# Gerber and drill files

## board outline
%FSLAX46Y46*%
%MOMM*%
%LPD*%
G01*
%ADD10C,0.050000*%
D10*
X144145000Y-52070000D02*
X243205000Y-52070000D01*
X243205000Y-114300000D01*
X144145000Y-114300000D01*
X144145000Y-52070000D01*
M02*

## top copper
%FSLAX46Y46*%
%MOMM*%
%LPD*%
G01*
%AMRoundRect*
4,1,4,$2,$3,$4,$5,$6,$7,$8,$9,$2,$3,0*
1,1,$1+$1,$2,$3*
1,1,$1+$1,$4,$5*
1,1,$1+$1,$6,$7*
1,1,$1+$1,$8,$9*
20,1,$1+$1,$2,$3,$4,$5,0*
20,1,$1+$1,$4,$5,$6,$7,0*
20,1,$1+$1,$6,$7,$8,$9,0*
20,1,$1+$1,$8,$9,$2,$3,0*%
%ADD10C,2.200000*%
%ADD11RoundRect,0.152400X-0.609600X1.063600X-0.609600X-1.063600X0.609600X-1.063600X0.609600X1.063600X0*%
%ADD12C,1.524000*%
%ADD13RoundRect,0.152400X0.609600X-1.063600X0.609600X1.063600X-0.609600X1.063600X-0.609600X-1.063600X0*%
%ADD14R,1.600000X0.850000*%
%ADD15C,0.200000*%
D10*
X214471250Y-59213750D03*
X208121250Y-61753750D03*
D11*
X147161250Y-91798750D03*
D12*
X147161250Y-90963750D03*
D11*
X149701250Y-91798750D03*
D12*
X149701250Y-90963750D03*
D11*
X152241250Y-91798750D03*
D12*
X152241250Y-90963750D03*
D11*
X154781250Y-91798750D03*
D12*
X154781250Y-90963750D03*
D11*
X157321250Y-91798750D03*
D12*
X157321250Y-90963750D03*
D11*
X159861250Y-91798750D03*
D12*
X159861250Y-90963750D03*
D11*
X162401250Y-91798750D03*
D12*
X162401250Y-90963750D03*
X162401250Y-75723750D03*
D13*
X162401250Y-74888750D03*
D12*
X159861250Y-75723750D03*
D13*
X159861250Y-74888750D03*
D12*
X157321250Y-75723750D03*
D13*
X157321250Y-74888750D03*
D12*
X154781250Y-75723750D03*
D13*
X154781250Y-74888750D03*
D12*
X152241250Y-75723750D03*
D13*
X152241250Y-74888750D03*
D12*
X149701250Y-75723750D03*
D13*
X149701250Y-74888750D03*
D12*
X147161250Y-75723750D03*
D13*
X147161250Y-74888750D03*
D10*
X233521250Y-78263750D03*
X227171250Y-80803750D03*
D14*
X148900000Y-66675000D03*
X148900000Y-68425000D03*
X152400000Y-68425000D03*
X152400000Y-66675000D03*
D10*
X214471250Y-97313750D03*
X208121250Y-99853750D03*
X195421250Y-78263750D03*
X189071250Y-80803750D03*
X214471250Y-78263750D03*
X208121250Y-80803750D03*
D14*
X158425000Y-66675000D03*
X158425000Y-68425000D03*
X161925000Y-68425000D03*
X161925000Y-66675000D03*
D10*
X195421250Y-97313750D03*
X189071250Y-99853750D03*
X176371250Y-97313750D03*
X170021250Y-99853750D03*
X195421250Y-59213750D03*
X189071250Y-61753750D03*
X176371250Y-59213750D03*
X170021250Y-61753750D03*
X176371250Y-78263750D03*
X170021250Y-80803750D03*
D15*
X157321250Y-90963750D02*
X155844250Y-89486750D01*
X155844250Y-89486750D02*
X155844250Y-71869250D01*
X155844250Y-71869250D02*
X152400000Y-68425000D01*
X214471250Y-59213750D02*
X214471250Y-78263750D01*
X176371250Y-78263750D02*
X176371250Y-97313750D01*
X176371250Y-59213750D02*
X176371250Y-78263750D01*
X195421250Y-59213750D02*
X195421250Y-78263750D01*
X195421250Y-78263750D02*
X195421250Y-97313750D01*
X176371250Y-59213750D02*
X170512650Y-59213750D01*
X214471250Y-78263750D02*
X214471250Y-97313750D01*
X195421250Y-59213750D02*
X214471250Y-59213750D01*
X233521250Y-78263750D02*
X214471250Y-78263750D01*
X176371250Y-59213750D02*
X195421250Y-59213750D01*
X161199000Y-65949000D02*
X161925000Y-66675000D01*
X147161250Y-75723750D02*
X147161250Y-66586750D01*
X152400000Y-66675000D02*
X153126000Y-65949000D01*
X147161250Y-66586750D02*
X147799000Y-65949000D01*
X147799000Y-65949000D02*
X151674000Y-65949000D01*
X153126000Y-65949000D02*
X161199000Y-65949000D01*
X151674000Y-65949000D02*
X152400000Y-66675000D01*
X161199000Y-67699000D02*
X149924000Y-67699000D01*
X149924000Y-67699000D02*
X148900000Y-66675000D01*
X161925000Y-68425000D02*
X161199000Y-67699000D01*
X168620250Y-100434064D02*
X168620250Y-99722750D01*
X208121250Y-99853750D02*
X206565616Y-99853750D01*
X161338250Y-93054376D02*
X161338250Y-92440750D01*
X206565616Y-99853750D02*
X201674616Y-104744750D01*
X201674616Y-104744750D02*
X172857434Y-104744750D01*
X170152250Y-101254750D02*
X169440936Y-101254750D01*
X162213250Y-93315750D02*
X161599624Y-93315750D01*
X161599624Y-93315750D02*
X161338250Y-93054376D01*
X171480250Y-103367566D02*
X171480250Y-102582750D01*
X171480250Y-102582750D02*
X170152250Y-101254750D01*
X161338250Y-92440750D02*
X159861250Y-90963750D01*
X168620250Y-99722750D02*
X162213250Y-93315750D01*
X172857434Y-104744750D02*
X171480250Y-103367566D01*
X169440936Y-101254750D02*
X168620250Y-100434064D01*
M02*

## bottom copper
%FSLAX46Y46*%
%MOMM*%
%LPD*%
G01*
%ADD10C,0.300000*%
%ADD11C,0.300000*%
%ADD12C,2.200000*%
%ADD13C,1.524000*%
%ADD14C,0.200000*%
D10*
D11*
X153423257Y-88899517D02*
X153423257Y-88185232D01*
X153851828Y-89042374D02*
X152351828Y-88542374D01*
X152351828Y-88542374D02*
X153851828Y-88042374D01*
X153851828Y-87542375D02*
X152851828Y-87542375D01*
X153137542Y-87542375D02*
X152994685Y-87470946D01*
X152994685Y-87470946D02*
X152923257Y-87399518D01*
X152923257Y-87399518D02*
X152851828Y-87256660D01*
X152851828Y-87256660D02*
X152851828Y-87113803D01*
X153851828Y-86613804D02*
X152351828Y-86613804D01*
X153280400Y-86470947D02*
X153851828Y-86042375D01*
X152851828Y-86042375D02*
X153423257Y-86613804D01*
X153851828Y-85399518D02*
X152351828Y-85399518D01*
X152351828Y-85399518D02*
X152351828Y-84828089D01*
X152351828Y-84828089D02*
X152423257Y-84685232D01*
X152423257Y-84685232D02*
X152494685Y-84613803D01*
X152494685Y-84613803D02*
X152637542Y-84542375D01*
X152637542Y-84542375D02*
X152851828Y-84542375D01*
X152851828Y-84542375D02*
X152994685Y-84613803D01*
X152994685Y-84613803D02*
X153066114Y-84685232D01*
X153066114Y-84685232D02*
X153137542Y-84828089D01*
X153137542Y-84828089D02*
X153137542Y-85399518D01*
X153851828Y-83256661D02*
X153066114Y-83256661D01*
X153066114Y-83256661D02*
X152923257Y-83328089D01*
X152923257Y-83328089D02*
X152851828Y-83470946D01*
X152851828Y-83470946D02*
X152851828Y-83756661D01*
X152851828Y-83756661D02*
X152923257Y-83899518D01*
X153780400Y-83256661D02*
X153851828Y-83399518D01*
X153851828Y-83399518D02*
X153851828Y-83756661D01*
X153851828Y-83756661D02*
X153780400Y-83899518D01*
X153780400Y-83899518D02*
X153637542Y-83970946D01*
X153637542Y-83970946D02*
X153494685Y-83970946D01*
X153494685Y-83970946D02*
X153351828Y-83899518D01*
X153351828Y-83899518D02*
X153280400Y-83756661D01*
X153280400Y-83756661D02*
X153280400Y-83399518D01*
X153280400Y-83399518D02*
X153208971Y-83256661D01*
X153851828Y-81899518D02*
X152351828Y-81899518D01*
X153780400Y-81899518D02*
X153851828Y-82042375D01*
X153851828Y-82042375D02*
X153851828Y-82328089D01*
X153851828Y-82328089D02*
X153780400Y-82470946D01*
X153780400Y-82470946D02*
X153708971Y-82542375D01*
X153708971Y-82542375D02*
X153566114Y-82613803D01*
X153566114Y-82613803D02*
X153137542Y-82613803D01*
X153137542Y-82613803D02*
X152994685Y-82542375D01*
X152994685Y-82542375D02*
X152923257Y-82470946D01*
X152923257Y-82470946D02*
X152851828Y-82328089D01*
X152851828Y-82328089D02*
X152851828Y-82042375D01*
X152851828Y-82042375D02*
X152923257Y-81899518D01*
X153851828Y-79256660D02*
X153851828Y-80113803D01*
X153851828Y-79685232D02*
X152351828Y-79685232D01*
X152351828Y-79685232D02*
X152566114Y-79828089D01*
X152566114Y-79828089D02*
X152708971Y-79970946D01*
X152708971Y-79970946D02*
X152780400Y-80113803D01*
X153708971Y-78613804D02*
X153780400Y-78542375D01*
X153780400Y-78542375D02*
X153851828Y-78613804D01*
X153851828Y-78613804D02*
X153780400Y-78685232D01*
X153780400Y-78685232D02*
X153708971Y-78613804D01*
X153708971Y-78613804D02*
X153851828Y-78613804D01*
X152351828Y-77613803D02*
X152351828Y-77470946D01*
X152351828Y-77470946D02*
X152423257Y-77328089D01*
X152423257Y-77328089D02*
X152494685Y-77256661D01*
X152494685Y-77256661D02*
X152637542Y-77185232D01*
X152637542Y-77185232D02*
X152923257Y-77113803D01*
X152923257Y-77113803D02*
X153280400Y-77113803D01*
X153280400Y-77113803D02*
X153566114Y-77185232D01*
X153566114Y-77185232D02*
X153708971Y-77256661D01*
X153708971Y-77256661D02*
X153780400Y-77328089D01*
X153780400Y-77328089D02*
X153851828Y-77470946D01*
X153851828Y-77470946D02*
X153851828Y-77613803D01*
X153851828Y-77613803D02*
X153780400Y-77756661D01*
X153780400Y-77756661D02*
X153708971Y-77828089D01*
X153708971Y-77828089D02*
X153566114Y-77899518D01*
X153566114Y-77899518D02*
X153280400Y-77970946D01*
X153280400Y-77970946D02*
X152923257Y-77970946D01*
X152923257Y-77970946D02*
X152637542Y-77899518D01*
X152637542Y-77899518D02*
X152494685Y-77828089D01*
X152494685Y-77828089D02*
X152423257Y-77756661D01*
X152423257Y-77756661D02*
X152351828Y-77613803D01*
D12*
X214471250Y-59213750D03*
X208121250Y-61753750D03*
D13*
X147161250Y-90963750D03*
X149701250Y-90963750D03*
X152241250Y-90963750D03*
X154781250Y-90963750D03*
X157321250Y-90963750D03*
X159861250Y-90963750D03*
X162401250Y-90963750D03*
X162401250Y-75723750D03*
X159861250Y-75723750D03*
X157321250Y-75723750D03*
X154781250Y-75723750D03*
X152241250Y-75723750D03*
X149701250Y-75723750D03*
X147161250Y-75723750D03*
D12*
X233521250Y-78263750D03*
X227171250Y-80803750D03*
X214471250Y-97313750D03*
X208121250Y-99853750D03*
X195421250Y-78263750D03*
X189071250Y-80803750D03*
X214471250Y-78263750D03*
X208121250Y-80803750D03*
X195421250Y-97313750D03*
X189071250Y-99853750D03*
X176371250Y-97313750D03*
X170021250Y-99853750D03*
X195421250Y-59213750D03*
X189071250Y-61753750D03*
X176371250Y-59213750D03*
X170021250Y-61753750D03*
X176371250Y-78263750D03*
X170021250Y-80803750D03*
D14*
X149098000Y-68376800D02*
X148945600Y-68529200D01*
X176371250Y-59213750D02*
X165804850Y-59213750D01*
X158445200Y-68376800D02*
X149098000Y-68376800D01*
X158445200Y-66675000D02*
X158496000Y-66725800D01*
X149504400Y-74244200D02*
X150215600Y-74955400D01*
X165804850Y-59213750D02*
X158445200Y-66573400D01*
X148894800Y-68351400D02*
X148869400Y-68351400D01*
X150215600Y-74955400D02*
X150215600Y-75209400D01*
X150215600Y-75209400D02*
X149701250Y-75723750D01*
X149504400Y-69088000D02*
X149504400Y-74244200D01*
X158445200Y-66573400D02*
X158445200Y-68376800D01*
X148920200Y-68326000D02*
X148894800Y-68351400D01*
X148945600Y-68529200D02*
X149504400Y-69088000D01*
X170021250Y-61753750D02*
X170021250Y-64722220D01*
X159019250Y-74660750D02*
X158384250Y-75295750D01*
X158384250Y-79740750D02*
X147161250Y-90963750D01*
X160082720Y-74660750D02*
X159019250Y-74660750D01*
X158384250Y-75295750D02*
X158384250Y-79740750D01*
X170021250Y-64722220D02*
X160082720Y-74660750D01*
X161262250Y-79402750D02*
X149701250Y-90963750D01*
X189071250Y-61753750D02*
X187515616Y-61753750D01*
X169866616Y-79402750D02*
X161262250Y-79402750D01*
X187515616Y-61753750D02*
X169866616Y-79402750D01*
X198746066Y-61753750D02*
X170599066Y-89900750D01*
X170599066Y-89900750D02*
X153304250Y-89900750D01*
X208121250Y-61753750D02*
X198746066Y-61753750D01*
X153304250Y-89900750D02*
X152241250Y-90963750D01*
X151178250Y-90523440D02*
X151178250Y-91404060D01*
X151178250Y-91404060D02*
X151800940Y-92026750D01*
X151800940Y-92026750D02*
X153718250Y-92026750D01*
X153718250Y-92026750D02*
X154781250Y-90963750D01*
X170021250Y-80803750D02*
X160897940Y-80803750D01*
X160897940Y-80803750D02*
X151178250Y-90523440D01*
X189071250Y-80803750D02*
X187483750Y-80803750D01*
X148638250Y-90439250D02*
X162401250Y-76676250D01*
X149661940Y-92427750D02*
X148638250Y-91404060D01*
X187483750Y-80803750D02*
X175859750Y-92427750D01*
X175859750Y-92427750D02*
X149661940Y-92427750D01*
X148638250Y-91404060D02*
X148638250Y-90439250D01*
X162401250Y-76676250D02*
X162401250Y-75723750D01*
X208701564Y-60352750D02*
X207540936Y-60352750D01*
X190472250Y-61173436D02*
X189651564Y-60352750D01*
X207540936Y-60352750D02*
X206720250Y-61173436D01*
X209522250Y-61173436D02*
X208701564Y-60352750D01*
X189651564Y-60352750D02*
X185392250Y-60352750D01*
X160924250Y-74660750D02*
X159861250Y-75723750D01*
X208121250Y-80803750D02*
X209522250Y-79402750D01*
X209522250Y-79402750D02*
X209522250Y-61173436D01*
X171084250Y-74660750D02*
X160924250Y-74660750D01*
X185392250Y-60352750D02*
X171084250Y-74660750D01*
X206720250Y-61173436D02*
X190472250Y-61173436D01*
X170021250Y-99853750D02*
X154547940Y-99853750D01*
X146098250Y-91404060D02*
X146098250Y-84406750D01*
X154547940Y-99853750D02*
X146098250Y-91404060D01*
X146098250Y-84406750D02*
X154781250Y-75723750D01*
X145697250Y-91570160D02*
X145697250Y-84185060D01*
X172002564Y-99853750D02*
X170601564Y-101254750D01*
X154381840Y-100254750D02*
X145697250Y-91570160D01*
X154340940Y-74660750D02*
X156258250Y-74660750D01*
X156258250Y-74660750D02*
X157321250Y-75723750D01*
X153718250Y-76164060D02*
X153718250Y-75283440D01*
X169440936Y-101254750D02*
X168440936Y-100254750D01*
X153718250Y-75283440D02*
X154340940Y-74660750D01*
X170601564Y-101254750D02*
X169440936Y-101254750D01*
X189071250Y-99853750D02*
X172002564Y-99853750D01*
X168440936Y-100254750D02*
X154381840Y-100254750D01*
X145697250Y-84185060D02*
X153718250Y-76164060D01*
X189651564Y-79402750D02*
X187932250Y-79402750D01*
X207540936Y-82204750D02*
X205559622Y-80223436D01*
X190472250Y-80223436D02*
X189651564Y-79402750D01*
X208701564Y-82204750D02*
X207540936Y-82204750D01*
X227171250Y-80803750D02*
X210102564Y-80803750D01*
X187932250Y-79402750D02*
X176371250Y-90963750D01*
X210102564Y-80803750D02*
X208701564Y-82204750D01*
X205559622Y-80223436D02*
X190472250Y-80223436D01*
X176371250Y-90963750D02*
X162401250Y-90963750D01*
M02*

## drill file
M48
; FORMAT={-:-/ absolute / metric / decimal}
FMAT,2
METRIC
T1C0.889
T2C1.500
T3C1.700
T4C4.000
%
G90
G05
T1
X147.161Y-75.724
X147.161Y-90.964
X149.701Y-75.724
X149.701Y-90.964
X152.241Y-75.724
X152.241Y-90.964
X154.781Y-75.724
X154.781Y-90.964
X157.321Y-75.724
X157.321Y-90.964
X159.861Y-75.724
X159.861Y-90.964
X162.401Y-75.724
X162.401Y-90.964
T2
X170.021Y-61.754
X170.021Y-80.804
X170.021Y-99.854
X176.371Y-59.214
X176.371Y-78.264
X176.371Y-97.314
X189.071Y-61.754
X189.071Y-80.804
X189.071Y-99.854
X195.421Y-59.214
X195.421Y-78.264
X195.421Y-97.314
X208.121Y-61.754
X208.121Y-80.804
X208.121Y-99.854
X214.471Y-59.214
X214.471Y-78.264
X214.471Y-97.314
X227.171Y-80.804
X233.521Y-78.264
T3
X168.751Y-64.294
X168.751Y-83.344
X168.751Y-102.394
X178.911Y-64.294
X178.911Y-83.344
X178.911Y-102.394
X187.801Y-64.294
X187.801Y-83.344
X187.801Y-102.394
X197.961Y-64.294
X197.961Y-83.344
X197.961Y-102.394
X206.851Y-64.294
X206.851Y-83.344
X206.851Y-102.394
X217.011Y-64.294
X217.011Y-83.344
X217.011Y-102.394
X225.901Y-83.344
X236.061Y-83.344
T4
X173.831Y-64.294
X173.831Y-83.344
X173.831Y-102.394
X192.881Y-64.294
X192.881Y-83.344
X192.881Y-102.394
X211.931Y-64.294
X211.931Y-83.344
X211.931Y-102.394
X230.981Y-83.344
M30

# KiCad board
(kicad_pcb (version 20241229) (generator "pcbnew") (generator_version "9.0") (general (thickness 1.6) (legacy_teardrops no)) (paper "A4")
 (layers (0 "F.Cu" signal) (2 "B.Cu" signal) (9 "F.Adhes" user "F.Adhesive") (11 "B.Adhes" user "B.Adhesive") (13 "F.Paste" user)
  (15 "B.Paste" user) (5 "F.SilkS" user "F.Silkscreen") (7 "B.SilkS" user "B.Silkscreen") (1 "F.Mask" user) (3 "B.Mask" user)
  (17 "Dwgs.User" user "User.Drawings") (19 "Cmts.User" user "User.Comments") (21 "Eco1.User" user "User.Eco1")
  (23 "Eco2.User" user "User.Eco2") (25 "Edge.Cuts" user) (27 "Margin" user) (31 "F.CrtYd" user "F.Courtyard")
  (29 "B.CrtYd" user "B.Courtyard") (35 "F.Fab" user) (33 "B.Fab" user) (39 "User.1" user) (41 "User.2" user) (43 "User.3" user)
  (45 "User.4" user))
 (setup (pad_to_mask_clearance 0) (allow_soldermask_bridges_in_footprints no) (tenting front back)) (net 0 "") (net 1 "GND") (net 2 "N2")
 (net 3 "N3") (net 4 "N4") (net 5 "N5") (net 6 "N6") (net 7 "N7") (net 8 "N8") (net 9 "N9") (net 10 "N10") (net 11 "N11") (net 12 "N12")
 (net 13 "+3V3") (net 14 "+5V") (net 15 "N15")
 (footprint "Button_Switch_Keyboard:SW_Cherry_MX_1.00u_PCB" (layer "F.Cu") (at 214.47125 59.21375)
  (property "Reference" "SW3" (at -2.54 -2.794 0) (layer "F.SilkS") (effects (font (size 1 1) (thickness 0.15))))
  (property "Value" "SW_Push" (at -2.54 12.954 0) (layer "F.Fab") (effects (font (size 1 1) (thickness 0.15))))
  (pad "" np_thru_hole circle (at -7.62 5.08) (size 1.7 1.7) (drill 1.7) (layers "*.Cu" "*.Mask"))
  (pad "" np_thru_hole circle (at -2.54 5.08) (size 4 4) (drill 4) (layers "*.Cu" "*.Mask"))
  (pad "" np_thru_hole circle (at 2.54 5.08) (size 1.7 1.7) (drill 1.7) (layers "*.Cu" "*.Mask"))
  (pad "1" thru_hole circle (at 0 0) (size 2.2 2.2) (drill 1.5) (layers "*.Cu" "*.Mask") (remove_unused_layers no) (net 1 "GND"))
  (pad "2" thru_hole circle (at -6.35 2.54) (size 2.2 2.2) (drill 1.5) (layers "*.Cu" "*.Mask") (remove_unused_layers no) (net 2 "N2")))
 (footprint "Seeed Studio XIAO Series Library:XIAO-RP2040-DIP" (layer "F.Cu") (at 154.78125 83.34375 90)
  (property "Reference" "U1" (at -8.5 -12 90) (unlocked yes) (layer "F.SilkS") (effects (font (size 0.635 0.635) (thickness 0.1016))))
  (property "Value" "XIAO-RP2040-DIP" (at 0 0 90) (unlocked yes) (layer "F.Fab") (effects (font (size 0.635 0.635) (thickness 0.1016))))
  (pad "1" smd roundrect (at -8.455 -7.62 270) (size 2.432 1.524) (layers "F.Cu" "F.Mask") (roundrect_rratio 0.1) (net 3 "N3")
   (thermal_bridge_angle 45))
  (pad "1" thru_hole circle (at -7.62 -7.62 270) (size 1.524 1.524) (drill 0.889) (layers "*.Cu" "*.Mask") (remove_unused_layers no)
   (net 3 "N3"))
  (pad "2" smd roundrect (at -8.455 -5.08 270) (size 2.432 1.524) (layers "F.Cu" "F.Mask") (roundrect_rratio 0.1) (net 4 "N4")
   (thermal_bridge_angle 45))
  (pad "2" thru_hole circle (at -7.62 -5.08 270) (size 1.524 1.524) (drill 0.889) (layers "*.Cu" "*.Mask") (remove_unused_layers no)
   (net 4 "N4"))
  (pad "3" smd roundrect (at -8.455 -2.54 270) (size 2.432 1.524) (layers "F.Cu" "F.Mask") (roundrect_rratio 0.1) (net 2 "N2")
   (thermal_bridge_angle 45))
  (pad "3" thru_hole circle (at -7.62 -2.54 270) (size 1.524 1.524) (drill 0.889) (layers "*.Cu" "*.Mask") (remove_unused_layers no)
   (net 2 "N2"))
  (pad "4" smd roundrect (at -8.455 0 270) (size 2.432 1.524) (layers "F.Cu" "F.Mask") (roundrect_rratio 0.1) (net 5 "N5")
   (thermal_bridge_angle 45))
  (pad "4" thru_hole circle (at -7.62 0 270) (size 1.524 1.524) (drill 0.889) (layers "*.Cu" "*.Mask") (remove_unused_layers no)
   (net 5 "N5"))
  (pad "5" smd roundrect (at -8.455 2.54 270) (size 2.432 1.524) (layers "F.Cu" "F.Mask") (roundrect_rratio 0.1) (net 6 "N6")
   (thermal_bridge_angle 45))
  (pad "5" thru_hole circle (at -7.62 2.54 270) (size 1.524 1.524) (drill 0.889) (layers "*.Cu" "*.Mask") (remove_unused_layers no)
   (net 6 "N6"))
  (pad "6" smd roundrect (at -8.455 5.08 270) (size 2.432 1.524) (layers "F.Cu" "F.Mask") (roundrect_rratio 0.1) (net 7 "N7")
   (thermal_bridge_angle 45))
  (pad "6" thru_hole circle (at -7.62 5.08 270) (size 1.524 1.524) (drill 0.889) (layers "*.Cu" "*.Mask") (remove_unused_layers no)
   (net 7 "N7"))
  (pad "7" smd roundrect (at -8.455 7.62 270) (size 2.432 1.524) (layers "F.Cu" "F.Mask") (roundrect_rratio 0.1) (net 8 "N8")
   (thermal_bridge_angle 45))
  (pad "7" thru_hole circle (at -7.62 7.62 270) (size 1.524 1.524) (drill 0.889) (layers "*.Cu" "*.Mask") (remove_unused_layers no)
   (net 8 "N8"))
  (pad "8" thru_hole circle (at 7.62 7.62 90) (size 1.524 1.524) (drill 0.889) (layers "*.Cu" "*.Mask") (remove_unused_layers no)
   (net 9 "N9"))
  (pad "8" smd roundrect (at 8.455 7.62 90) (size 2.432 1.524) (layers "F.Cu" "F.Mask") (roundrect_rratio 0.1) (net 9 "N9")
   (thermal_bridge_angle 45))
  (pad "9" thru_hole circle (at 7.62 5.08 90) (size 1.524 1.524) (drill 0.889) (layers "*.Cu" "*.Mask") (remove_unused_layers no)
   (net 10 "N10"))
  (pad "9" smd roundrect (at 8.455 5.08 90) (size 2.432 1.524) (layers "F.Cu" "F.Mask") (roundrect_rratio 0.1) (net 10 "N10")
   (thermal_bridge_angle 45))
  (pad "10" thru_hole circle (at 7.62 2.54 90) (size 1.524 1.524) (drill 0.889) (layers "*.Cu" "*.Mask") (remove_unused_layers no)
   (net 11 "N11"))
  (pad "10" smd roundrect (at 8.455 2.54 90) (size 2.432 1.524) (layers "F.Cu" "F.Mask") (roundrect_rratio 0.1) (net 11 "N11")
   (thermal_bridge_angle 45))
  (pad "11" thru_hole circle (at 7.62 0 90) (size 1.524 1.524) (drill 0.889) (layers "*.Cu" "*.Mask") (remove_unused_layers no)
   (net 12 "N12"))
  (pad "11" smd roundrect (at 8.455 0 90) (size 2.432 1.524) (layers "F.Cu" "F.Mask") (roundrect_rratio 0.1) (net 12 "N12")
   (thermal_bridge_angle 45))
  (pad "12" thru_hole circle (at 7.62 -2.54 90) (size 1.524 1.524) (drill 0.889) (layers "*.Cu" "*.Mask") (remove_unused_layers no)
   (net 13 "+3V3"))
  (pad "12" smd roundrect (at 8.455 -2.54 90) (size 2.432 1.524) (layers "F.Cu" "F.Mask") (roundrect_rratio 0.1) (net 13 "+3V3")
   (thermal_bridge_angle 45))
  (pad "13" thru_hole circle (at 7.62 -5.08 90) (size 1.524 1.524) (drill 0.889) (layers "*.Cu" "*.Mask") (remove_unused_layers no)
   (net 1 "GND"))
  (pad "13" smd roundrect (at 8.455 -5.08 90) (size 2.432 1.524) (layers "F.Cu" "F.Mask") (roundrect_rratio 0.1) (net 1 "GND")
   (thermal_bridge_angle 45))
  (pad "14" thru_hole circle (at 7.62 -7.62 90) (size 1.524 1.524) (drill 0.889) (layers "*.Cu" "*.Mask") (remove_unused_layers no)
   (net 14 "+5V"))
  (pad "14" smd roundrect (at 8.455 -7.62 90) (size 2.432 1.524) (layers "F.Cu" "F.Mask") (roundrect_rratio 0.1) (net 14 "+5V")
   (thermal_bridge_angle 45)))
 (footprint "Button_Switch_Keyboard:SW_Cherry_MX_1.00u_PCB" (layer "F.Cu") (at 233.52125 78.26375)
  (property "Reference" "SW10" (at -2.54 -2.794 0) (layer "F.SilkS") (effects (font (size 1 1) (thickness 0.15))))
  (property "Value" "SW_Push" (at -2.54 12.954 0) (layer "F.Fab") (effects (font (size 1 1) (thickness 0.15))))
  (pad "" np_thru_hole circle (at -7.62 5.08) (size 1.7 1.7) (drill 1.7) (layers "*.Cu" "*.Mask"))
  (pad "" np_thru_hole circle (at -2.54 5.08) (size 4 4) (drill 4) (layers "*.Cu" "*.Mask"))
  (pad "" np_thru_hole circle (at 2.54 5.08) (size 1.7 1.7) (drill 1.7) (layers "*.Cu" "*.Mask"))
  (pad "1" thru_hole circle (at 0 0) (size 2.2 2.2) (drill 1.5) (layers "*.Cu" "*.Mask") (remove_unused_layers no) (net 1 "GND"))
  (pad "2" thru_hole circle (at -6.35 2.54) (size 2.2 2.2) (drill 1.5) (layers "*.Cu" "*.Mask") (remove_unused_layers no) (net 8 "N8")))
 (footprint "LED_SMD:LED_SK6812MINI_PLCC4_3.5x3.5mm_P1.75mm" (layer "F.Cu") (at 150.65 67.55)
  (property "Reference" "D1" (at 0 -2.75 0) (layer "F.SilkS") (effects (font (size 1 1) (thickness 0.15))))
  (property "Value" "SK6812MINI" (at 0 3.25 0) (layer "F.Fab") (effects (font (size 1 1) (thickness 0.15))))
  (pad "1" smd rect (at -1.75 -0.875) (size 1.6 0.85) (layers "F.Cu" "F.Mask" "F.Paste") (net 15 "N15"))
  (pad "2" smd rect (at -1.75 0.875) (size 1.6 0.85) (layers "F.Cu" "F.Mask" "F.Paste") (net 1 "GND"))
  (pad "3" smd rect (at 1.75 0.875) (size 1.6 0.85) (layers "F.Cu" "F.Mask" "F.Paste") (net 6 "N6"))
  (pad "4" smd rect (at 1.75 -0.875) (size 1.6 0.85) (layers "F.Cu" "F.Mask" "F.Paste") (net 14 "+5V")))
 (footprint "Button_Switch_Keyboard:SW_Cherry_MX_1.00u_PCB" (layer "F.Cu") (at 214.47125 97.31375)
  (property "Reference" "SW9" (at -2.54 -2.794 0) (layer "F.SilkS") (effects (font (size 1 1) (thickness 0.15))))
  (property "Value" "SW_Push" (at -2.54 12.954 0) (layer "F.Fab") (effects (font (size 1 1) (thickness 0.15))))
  (pad "" np_thru_hole circle (at -7.62 5.08) (size 1.7 1.7) (drill 1.7) (layers "*.Cu" "*.Mask"))
  (pad "" np_thru_hole circle (at -2.54 5.08) (size 4 4) (drill 4) (layers "*.Cu" "*.Mask"))
  (pad "" np_thru_hole circle (at 2.54 5.08) (size 1.7 1.7) (drill 1.7) (layers "*.Cu" "*.Mask"))
  (pad "1" thru_hole circle (at 0 0) (size 2.2 2.2) (drill 1.5) (layers "*.Cu" "*.Mask") (remove_unused_layers no) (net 1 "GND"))
  (pad "2" thru_hole circle (at -6.35 2.54) (size 2.2 2.2) (drill 1.5) (layers "*.Cu" "*.Mask") (remove_unused_layers no) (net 7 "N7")))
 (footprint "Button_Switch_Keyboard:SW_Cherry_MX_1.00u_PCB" (layer "F.Cu") (at 195.42125 78.26375)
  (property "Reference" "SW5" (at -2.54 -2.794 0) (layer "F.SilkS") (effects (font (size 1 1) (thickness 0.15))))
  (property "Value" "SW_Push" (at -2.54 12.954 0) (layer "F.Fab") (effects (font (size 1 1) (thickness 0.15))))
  (pad "" np_thru_hole circle (at -7.62 5.08) (size 1.7 1.7) (drill 1.7) (layers "*.Cu" "*.Mask"))
  (pad "" np_thru_hole circle (at -2.54 5.08) (size 4 4) (drill 4) (layers "*.Cu" "*.Mask"))
  (pad "" np_thru_hole circle (at 2.54 5.08) (size 1.7 1.7) (drill 1.7) (layers "*.Cu" "*.Mask"))
  (pad "1" thru_hole circle (at 0 0) (size 2.2 2.2) (drill 1.5) (layers "*.Cu" "*.Mask") (remove_unused_layers no) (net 1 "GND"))
  (pad "2" thru_hole circle (at -6.35 2.54) (size 2.2 2.2) (drill 1.5) (layers "*.Cu" "*.Mask") (remove_unused_layers no) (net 9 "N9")))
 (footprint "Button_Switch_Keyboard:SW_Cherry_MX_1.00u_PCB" (layer "F.Cu") (at 214.47125 78.26375)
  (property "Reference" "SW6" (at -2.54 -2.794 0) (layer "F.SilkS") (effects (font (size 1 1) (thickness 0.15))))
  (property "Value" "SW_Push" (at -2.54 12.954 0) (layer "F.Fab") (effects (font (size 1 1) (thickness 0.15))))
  (pad "" np_thru_hole circle (at -7.62 5.08) (size 1.7 1.7) (drill 1.7) (layers "*.Cu" "*.Mask"))
  (pad "" np_thru_hole circle (at -2.54 5.08) (size 4 4) (drill 4) (layers "*.Cu" "*.Mask"))
  (pad "" np_thru_hole circle (at 2.54 5.08) (size 1.7 1.7) (drill 1.7) (layers "*.Cu" "*.Mask"))
  (pad "1" thru_hole circle (at 0 0) (size 2.2 2.2) (drill 1.5) (layers "*.Cu" "*.Mask") (remove_unused_layers no) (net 1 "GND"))
  (pad "2" thru_hole circle (at -6.35 2.54) (size 2.2 2.2) (drill 1.5) (layers "*.Cu" "*.Mask") (remove_unused_layers no) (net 10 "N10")))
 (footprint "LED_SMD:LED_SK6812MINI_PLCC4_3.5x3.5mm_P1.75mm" (layer "F.Cu") (at 160.175 67.55)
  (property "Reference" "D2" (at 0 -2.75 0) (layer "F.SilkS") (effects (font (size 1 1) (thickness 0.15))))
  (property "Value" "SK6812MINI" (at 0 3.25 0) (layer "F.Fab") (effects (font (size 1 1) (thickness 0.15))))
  (pad "1" smd rect (at -1.75 -0.875) (size 1.6 0.85) (layers "F.Cu" "F.Mask" "F.Paste") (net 1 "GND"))
  (pad "2" smd rect (at -1.75 0.875) (size 1.6 0.85) (layers "F.Cu" "F.Mask" "F.Paste") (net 1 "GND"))
  (pad "3" smd rect (at 1.75 0.875) (size 1.6 0.85) (layers "F.Cu" "F.Mask" "F.Paste") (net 15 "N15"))
  (pad "4" smd rect (at 1.75 -0.875) (size 1.6 0.85) (layers "F.Cu" "F.Mask" "F.Paste") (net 14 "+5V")))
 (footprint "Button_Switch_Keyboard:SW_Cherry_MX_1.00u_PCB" (layer "F.Cu") (at 195.42125 97.31375)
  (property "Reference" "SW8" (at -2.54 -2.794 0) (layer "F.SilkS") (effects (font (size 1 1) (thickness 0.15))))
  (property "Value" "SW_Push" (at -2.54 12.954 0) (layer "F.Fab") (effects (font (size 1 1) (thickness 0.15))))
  (pad "" np_thru_hole circle (at -7.62 5.08) (size 1.7 1.7) (drill 1.7) (layers "*.Cu" "*.Mask"))
  (pad "" np_thru_hole circle (at -2.54 5.08) (size 4 4) (drill 4) (layers "*.Cu" "*.Mask"))
  (pad "" np_thru_hole circle (at 2.54 5.08) (size 1.7 1.7) (drill 1.7) (layers "*.Cu" "*.Mask"))
  (pad "1" thru_hole circle (at 0 0) (size 2.2 2.2) (drill 1.5) (layers "*.Cu" "*.Mask") (remove_unused_layers no) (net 1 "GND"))
  (pad "2" thru_hole circle (at -6.35 2.54) (size 2.2 2.2) (drill 1.5) (layers "*.Cu" "*.Mask") (remove_unused_layers no) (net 11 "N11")))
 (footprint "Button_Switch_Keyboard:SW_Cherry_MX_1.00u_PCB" (layer "F.Cu") (at 176.37125 97.31375)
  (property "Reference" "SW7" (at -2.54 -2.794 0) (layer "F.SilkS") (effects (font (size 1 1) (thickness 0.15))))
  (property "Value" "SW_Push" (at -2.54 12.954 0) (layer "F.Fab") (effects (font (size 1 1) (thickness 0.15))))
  (pad "" np_thru_hole circle (at -7.62 5.08) (size 1.7 1.7) (drill 1.7) (layers "*.Cu" "*.Mask"))
  (pad "" np_thru_hole circle (at -2.54 5.08) (size 4 4) (drill 4) (layers "*.Cu" "*.Mask"))
  (pad "" np_thru_hole circle (at 2.54 5.08) (size 1.7 1.7) (drill 1.7) (layers "*.Cu" "*.Mask"))
  (pad "1" thru_hole circle (at 0 0) (size 2.2 2.2) (drill 1.5) (layers "*.Cu" "*.Mask") (remove_unused_layers no) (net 1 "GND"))
  (pad "2" thru_hole circle (at -6.35 2.54) (size 2.2 2.2) (drill 1.5) (layers "*.Cu" "*.Mask") (remove_unused_layers no) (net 12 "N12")))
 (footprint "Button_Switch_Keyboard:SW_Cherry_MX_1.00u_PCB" (layer "F.Cu") (at 195.42125 59.21375)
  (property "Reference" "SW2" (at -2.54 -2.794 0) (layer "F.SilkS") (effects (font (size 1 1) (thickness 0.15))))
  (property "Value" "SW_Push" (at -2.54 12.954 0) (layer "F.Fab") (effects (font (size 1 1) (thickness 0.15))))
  (pad "" np_thru_hole circle (at -7.62 5.08) (size 1.7 1.7) (drill 1.7) (layers "*.Cu" "*.Mask"))
  (pad "" np_thru_hole circle (at -2.54 5.08) (size 4 4) (drill 4) (layers "*.Cu" "*.Mask"))
  (pad "" np_thru_hole circle (at 2.54 5.08) (size 1.7 1.7) (drill 1.7) (layers "*.Cu" "*.Mask"))
  (pad "1" thru_hole circle (at 0 0) (size 2.2 2.2) (drill 1.5) (layers "*.Cu" "*.Mask") (remove_unused_layers no) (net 1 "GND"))
  (pad "2" thru_hole circle (at -6.35 2.54) (size 2.2 2.2) (drill 1.5) (layers "*.Cu" "*.Mask") (remove_unused_layers no) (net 4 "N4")))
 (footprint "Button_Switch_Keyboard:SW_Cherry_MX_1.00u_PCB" (layer "F.Cu") (at 176.37125 59.21375)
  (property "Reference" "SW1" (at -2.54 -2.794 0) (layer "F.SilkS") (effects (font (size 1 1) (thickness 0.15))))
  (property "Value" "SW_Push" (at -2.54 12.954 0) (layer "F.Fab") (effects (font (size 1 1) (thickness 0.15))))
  (pad "" np_thru_hole circle (at -7.62 5.08) (size 1.7 1.7) (drill 1.7) (layers "*.Cu" "*.Mask"))
  (pad "" np_thru_hole circle (at -2.54 5.08) (size 4 4) (drill 4) (layers "*.Cu" "*.Mask"))
  (pad "" np_thru_hole circle (at 2.54 5.08) (size 1.7 1.7) (drill 1.7) (layers "*.Cu" "*.Mask"))
  (pad "1" thru_hole circle (at 0 0) (size 2.2 2.2) (drill 1.5) (layers "*.Cu" "*.Mask") (remove_unused_layers no) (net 1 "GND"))
  (pad "2" thru_hole circle (at -6.35 2.54) (size 2.2 2.2) (drill 1.5) (layers "*.Cu" "*.Mask") (remove_unused_layers no) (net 3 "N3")))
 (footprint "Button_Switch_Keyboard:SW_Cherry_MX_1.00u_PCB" (layer "F.Cu") (at 176.37125 78.26375)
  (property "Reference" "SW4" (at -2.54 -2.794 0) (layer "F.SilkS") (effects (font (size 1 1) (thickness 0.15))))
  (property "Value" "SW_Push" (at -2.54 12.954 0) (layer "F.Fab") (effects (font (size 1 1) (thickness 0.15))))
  (pad "" np_thru_hole circle (at -7.62 5.08) (size 1.7 1.7) (drill 1.7) (layers "*.Cu" "*.Mask"))
  (pad "" np_thru_hole circle (at -2.54 5.08) (size 4 4) (drill 4) (layers "*.Cu" "*.Mask"))
  (pad "" np_thru_hole circle (at 2.54 5.08) (size 1.7 1.7) (drill 1.7) (layers "*.Cu" "*.Mask"))
  (pad "1" thru_hole circle (at 0 0) (size 2.2 2.2) (drill 1.5) (layers "*.Cu" "*.Mask") (remove_unused_layers no) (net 1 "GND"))
  (pad "2" thru_hole circle (at -6.35 2.54) (size 2.2 2.2) (drill 1.5) (layers "*.Cu" "*.Mask") (remove_unused_layers no) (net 5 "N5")))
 (gr_rect (start 144.145 52.07) (end 243.205 114.3) (stroke (width 0.05) (type default)) (fill no) (layer "Edge.Cuts"))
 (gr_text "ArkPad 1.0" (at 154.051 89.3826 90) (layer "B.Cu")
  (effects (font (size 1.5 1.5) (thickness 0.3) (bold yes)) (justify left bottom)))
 (segment (start 157.32125 90.96375) (end 155.84425 89.48675) (width 0.2) (layer "F.Cu") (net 6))
 (segment (start 155.84425 89.48675) (end 155.84425 71.86925) (width 0.2) (layer "F.Cu") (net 6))
 (segment (start 155.84425 71.86925) (end 152.4 68.425) (width 0.2) (layer "F.Cu") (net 6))
 (segment (start 214.47125 59.21375) (end 214.47125 78.26375) (width 0.2) (layer "F.Cu") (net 1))
 (segment (start 176.37125 78.26375) (end 176.37125 97.31375) (width 0.2) (layer "F.Cu") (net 1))
 (segment (start 176.37125 59.21375) (end 176.37125 78.26375) (width 0.2) (layer "F.Cu") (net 1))
 (segment (start 195.42125 59.21375) (end 195.42125 78.26375) (width 0.2) (layer "F.Cu") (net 1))
 (segment (start 195.42125 78.26375) (end 195.42125 97.31375) (width 0.2) (layer "F.Cu") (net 1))
 (segment (start 176.37125 59.21375) (end 170.51265 59.21375) (width 0.2) (layer "F.Cu") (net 1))
 (segment (start 214.47125 78.26375) (end 214.47125 97.31375) (width 0.2) (layer "F.Cu") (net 1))
 (segment (start 195.42125 59.21375) (end 214.47125 59.21375) (width 0.2) (layer "F.Cu") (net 1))
 (segment (start 233.52125 78.26375) (end 214.47125 78.26375) (width 0.2) (layer "F.Cu") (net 1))
 (segment (start 176.37125 59.21375) (end 195.42125 59.21375) (width 0.2) (layer "F.Cu") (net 1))
 (segment (start 149.098 68.3768) (end 148.9456 68.5292) (width 0.2) (layer "B.Cu") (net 1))
 (segment (start 176.37125 59.21375) (end 165.80485 59.21375) (width 0.2) (layer "B.Cu") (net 1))
 (segment (start 158.4452 68.3768) (end 149.098 68.3768) (width 0.2) (layer "B.Cu") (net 1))
 (segment (start 158.4452 66.675) (end 158.496 66.7258) (width 0.2) (layer "B.Cu") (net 1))
 (segment (start 149.5044 74.2442) (end 150.2156 74.9554) (width 0.2) (layer "B.Cu") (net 1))
 (segment (start 165.80485 59.21375) (end 158.4452 66.5734) (width 0.2) (layer "B.Cu") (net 1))
 (segment (start 148.8948 68.3514) (end 148.8694 68.3514) (width 0.2) (layer "B.Cu") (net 1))
 (segment (start 150.2156 74.9554) (end 150.2156 75.2094) (width 0.2) (layer "B.Cu") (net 1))
 (segment (start 150.2156 75.2094) (end 149.70125 75.72375) (width 0.2) (layer "B.Cu") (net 1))
 (segment (start 149.5044 69.088) (end 149.5044 74.2442) (width 0.2) (layer "B.Cu") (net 1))
 (segment (start 158.4452 66.5734) (end 158.4452 68.3768) (width 0.2) (layer "B.Cu") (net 1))
 (segment (start 148.9202 68.326) (end 148.8948 68.3514) (width 0.2) (layer "B.Cu") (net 1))
 (segment (start 148.9456 68.5292) (end 149.5044 69.088) (width 0.2) (layer "B.Cu") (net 1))
 (segment (start 161.199 65.949) (end 161.925 66.675) (width 0.2) (layer "F.Cu") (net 14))
 (segment (start 147.16125 75.72375) (end 147.16125 66.58675) (width 0.2) (layer "F.Cu") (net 14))
 (segment (start 152.4 66.675) (end 153.126 65.949) (width 0.2) (layer "F.Cu") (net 14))
 (segment (start 147.16125 66.58675) (end 147.799 65.949) (width 0.2) (layer "F.Cu") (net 14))
 (segment (start 147.799 65.949) (end 151.674 65.949) (width 0.2) (layer "F.Cu") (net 14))
 (segment (start 153.126 65.949) (end 161.199 65.949) (width 0.2) (layer "F.Cu") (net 14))
 (segment (start 151.674 65.949) (end 152.4 66.675) (width 0.2) (layer "F.Cu") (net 14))
 (segment (start 161.199 67.699) (end 149.924 67.699) (width 0.2) (layer "F.Cu") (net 15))
 (segment (start 149.924 67.699) (end 148.9 66.675) (width 0.2) (layer "F.Cu") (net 15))
 (segment (start 161.925 68.425) (end 161.199 67.699) (width 0.2) (layer "F.Cu") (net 15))
 (segment (start 170.02125 61.75375) (end 170.02125 64.72222) (width 0.2) (layer "B.Cu") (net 3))
 (segment (start 159.01925 74.66075) (end 158.38425 75.29575) (width 0.2) (layer "B.Cu") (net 3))
 (segment (start 158.38425 79.74075) (end 147.16125 90.96375) (width 0.2) (layer "B.Cu") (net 3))
 (segment (start 160.08272 74.66075) (end 159.01925 74.66075) (width 0.2) (layer "B.Cu") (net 3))
 (segment (start 158.38425 75.29575) (end 158.38425 79.74075) (width 0.2) (layer "B.Cu") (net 3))
 (segment (start 170.02125 64.72222) (end 160.08272 74.66075) (width 0.2) (layer "B.Cu") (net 3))
 (segment (start 161.26225 79.40275) (end 149.70125 90.96375) (width 0.2) (layer "B.Cu") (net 4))
 (segment (start 189.07125 61.75375) (end 187.515616 61.75375) (width 0.2) (layer "B.Cu") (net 4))
 (segment (start 169.866616 79.40275) (end 161.26225 79.40275) (width 0.2) (layer "B.Cu") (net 4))
 (segment (start 187.515616 61.75375) (end 169.866616 79.40275) (width 0.2) (layer "B.Cu") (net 4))
 (segment (start 198.746066 61.75375) (end 170.599066 89.90075) (width 0.2) (layer "B.Cu") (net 2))
 (segment (start 170.599066 89.90075) (end 153.30425 89.90075) (width 0.2) (layer "B.Cu") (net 2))
 (segment (start 208.12125 61.75375) (end 198.746066 61.75375) (width 0.2) (layer "B.Cu") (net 2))
 (segment (start 153.30425 89.90075) (end 152.24125 90.96375) (width 0.2) (layer "B.Cu") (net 2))
 (segment (start 151.17825 90.52344) (end 151.17825 91.40406) (width 0.2) (layer "B.Cu") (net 5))
 (segment (start 151.17825 91.40406) (end 151.80094 92.02675) (width 0.2) (layer "B.Cu") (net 5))
 (segment (start 151.80094 92.02675) (end 153.71825 92.02675) (width 0.2) (layer "B.Cu") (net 5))
 (segment (start 153.71825 92.02675) (end 154.78125 90.96375) (width 0.2) (layer "B.Cu") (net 5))
 (segment (start 170.02125 80.80375) (end 160.89794 80.80375) (width 0.2) (layer "B.Cu") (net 5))
 (segment (start 160.89794 80.80375) (end 151.17825 90.52344) (width 0.2) (layer "B.Cu") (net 5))
 (segment (start 189.07125 80.80375) (end 187.48375 80.80375) (width 0.2) (layer "B.Cu") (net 9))
 (segment (start 148.63825 90.43925) (end 162.40125 76.67625) (width 0.2) (layer "B.Cu") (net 9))
 (segment (start 149.66194 92.42775) (end 148.63825 91.40406) (width 0.2) (layer "B.Cu") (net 9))
 (segment (start 187.48375 80.80375) (end 175.85975 92.42775) (width 0.2) (layer "B.Cu") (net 9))
 (segment (start 175.85975 92.42775) (end 149.66194 92.42775) (width 0.2) (layer "B.Cu") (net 9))
 (segment (start 148.63825 91.40406) (end 148.63825 90.43925) (width 0.2) (layer "B.Cu") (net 9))
 (segment (start 162.40125 76.67625) (end 162.40125 75.72375) (width 0.2) (layer "B.Cu") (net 9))
 (segment (start 208.701564 60.35275) (end 207.540936 60.35275) (width 0.2) (layer "B.Cu") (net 10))
 (segment (start 190.47225 61.173436) (end 189.651564 60.35275) (width 0.2) (layer "B.Cu") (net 10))
 (segment (start 207.540936 60.35275) (end 206.72025 61.173436) (width 0.2) (layer "B.Cu") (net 10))
 (segment (start 209.52225 61.173436) (end 208.701564 60.35275) (width 0.2) (layer "B.Cu") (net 10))
 (segment (start 189.651564 60.35275) (end 185.39225 60.35275) (width 0.2) (layer "B.Cu") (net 10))
 (segment (start 160.92425 74.66075) (end 159.86125 75.72375) (width 0.2) (layer "B.Cu") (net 10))
 (segment (start 208.12125 80.80375) (end 209.52225 79.40275) (width 0.2) (layer "B.Cu") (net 10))
 (segment (start 209.52225 79.40275) (end 209.52225 61.173436) (width 0.2) (layer "B.Cu") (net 10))
 (segment (start 171.08425 74.66075) (end 160.92425 74.66075) (width 0.2) (layer "B.Cu") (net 10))
 (segment (start 185.39225 60.35275) (end 171.08425 74.66075) (width 0.2) (layer "B.Cu") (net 10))
 (segment (start 206.72025 61.173436) (end 190.47225 61.173436) (width 0.2) (layer "B.Cu") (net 10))
 (segment (start 170.02125 99.85375) (end 154.54794 99.85375) (width 0.2) (layer "B.Cu") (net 12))
 (segment (start 146.09825 91.40406) (end 146.09825 84.40675) (width 0.2) (layer "B.Cu") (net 12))
 (segment (start 154.54794 99.85375) (end 146.09825 91.40406) (width 0.2) (layer "B.Cu") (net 12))
 (segment (start 146.09825 84.40675) (end 154.78125 75.72375) (width 0.2) (layer "B.Cu") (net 12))
 (segment (start 145.69725 91.57016) (end 145.69725 84.18506) (width 0.2) (layer "B.Cu") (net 11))
 (segment (start 172.002564 99.85375) (end 170.601564 101.25475) (width 0.2) (layer "B.Cu") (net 11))
 (segment (start 154.38184 100.25475) (end 145.69725 91.57016) (width 0.2) (layer "B.Cu") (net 11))
 (segment (start 154.34094 74.66075) (end 156.25825 74.66075) (width 0.2) (layer "B.Cu") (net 11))
 (segment (start 156.25825 74.66075) (end 157.32125 75.72375) (width 0.2) (layer "B.Cu") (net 11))
 (segment (start 153.71825 76.16406) (end 153.71825 75.28344) (width 0.2) (layer "B.Cu") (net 11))
 (segment (start 169.440936 101.25475) (end 168.440936 100.25475) (width 0.2) (layer "B.Cu") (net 11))
 (segment (start 153.71825 75.28344) (end 154.34094 74.66075) (width 0.2) (layer "B.Cu") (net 11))
 (segment (start 170.601564 101.25475) (end 169.440936 101.25475) (width 0.2) (layer "B.Cu") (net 11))
 (segment (start 189.07125 99.85375) (end 172.002564 99.85375) (width 0.2) (layer "B.Cu") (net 11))
 (segment (start 168.440936 100.25475) (end 154.38184 100.25475) (width 0.2) (layer "B.Cu") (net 11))
 (segment (start 145.69725 84.18506) (end 153.71825 76.16406) (width 0.2) (layer "B.Cu") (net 11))
 (segment (start 168.62025 100.434064) (end 168.62025 99.72275) (width 0.2) (layer "F.Cu") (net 7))
 (segment (start 208.12125 99.85375) (end 206.565616 99.85375) (width 0.2) (layer "F.Cu") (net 7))
 (segment (start 161.33825 93.054376) (end 161.33825 92.44075) (width 0.2) (layer "F.Cu") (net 7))
 (segment (start 206.565616 99.85375) (end 201.674616 104.74475) (width 0.2) (layer "F.Cu") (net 7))
 (segment (start 201.674616 104.74475) (end 172.857434 104.74475) (width 0.2) (layer "F.Cu") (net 7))
 (segment (start 170.15225 101.25475) (end 169.440936 101.25475) (width 0.2) (layer "F.Cu") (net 7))
 (segment (start 162.21325 93.31575) (end 161.599624 93.31575) (width 0.2) (layer "F.Cu") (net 7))
 (segment (start 161.599624 93.31575) (end 161.33825 93.054376) (width 0.2) (layer "F.Cu") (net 7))
 (segment (start 171.48025 103.367566) (end 171.48025 102.58275) (width 0.2) (layer "F.Cu") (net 7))
 (segment (start 171.48025 102.58275) (end 170.15225 101.25475) (width 0.2) (layer "F.Cu") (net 7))
 (segment (start 161.33825 92.44075) (end 159.86125 90.96375) (width 0.2) (layer "F.Cu") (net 7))
 (segment (start 168.62025 99.72275) (end 162.21325 93.31575) (width 0.2) (layer "F.Cu") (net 7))
 (segment (start 172.857434 104.74475) (end 171.48025 103.367566) (width 0.2) (layer "F.Cu") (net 7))
 (segment (start 169.440936 101.25475) (end 168.62025 100.434064) (width 0.2) (layer "F.Cu") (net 7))
 (segment (start 189.651564 79.40275) (end 187.93225 79.40275) (width 0.2) (layer "B.Cu") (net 8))
 (segment (start 207.540936 82.20475) (end 205.559622 80.223436) (width 0.2) (layer "B.Cu") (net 8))
 (segment (start 190.47225 80.223436) (end 189.651564 79.40275) (width 0.2) (layer "B.Cu") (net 8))
 (segment (start 208.701564 82.20475) (end 207.540936 82.20475) (width 0.2) (layer "B.Cu") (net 8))
 (segment (start 227.17125 80.80375) (end 210.102564 80.80375) (width 0.2) (layer "B.Cu") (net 8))
 (segment (start 187.93225 79.40275) (end 176.37125 90.96375) (width 0.2) (layer "B.Cu") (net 8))
 (segment (start 210.102564 80.80375) (end 208.701564 82.20475) (width 0.2) (layer "B.Cu") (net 8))
 (segment (start 205.559622 80.223436) (end 190.47225 80.223436) (width 0.2) (layer "B.Cu") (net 8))
 (segment (start 176.37125 90.96375) (end 162.40125 90.96375) (width 0.2) (layer "B.Cu") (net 8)))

